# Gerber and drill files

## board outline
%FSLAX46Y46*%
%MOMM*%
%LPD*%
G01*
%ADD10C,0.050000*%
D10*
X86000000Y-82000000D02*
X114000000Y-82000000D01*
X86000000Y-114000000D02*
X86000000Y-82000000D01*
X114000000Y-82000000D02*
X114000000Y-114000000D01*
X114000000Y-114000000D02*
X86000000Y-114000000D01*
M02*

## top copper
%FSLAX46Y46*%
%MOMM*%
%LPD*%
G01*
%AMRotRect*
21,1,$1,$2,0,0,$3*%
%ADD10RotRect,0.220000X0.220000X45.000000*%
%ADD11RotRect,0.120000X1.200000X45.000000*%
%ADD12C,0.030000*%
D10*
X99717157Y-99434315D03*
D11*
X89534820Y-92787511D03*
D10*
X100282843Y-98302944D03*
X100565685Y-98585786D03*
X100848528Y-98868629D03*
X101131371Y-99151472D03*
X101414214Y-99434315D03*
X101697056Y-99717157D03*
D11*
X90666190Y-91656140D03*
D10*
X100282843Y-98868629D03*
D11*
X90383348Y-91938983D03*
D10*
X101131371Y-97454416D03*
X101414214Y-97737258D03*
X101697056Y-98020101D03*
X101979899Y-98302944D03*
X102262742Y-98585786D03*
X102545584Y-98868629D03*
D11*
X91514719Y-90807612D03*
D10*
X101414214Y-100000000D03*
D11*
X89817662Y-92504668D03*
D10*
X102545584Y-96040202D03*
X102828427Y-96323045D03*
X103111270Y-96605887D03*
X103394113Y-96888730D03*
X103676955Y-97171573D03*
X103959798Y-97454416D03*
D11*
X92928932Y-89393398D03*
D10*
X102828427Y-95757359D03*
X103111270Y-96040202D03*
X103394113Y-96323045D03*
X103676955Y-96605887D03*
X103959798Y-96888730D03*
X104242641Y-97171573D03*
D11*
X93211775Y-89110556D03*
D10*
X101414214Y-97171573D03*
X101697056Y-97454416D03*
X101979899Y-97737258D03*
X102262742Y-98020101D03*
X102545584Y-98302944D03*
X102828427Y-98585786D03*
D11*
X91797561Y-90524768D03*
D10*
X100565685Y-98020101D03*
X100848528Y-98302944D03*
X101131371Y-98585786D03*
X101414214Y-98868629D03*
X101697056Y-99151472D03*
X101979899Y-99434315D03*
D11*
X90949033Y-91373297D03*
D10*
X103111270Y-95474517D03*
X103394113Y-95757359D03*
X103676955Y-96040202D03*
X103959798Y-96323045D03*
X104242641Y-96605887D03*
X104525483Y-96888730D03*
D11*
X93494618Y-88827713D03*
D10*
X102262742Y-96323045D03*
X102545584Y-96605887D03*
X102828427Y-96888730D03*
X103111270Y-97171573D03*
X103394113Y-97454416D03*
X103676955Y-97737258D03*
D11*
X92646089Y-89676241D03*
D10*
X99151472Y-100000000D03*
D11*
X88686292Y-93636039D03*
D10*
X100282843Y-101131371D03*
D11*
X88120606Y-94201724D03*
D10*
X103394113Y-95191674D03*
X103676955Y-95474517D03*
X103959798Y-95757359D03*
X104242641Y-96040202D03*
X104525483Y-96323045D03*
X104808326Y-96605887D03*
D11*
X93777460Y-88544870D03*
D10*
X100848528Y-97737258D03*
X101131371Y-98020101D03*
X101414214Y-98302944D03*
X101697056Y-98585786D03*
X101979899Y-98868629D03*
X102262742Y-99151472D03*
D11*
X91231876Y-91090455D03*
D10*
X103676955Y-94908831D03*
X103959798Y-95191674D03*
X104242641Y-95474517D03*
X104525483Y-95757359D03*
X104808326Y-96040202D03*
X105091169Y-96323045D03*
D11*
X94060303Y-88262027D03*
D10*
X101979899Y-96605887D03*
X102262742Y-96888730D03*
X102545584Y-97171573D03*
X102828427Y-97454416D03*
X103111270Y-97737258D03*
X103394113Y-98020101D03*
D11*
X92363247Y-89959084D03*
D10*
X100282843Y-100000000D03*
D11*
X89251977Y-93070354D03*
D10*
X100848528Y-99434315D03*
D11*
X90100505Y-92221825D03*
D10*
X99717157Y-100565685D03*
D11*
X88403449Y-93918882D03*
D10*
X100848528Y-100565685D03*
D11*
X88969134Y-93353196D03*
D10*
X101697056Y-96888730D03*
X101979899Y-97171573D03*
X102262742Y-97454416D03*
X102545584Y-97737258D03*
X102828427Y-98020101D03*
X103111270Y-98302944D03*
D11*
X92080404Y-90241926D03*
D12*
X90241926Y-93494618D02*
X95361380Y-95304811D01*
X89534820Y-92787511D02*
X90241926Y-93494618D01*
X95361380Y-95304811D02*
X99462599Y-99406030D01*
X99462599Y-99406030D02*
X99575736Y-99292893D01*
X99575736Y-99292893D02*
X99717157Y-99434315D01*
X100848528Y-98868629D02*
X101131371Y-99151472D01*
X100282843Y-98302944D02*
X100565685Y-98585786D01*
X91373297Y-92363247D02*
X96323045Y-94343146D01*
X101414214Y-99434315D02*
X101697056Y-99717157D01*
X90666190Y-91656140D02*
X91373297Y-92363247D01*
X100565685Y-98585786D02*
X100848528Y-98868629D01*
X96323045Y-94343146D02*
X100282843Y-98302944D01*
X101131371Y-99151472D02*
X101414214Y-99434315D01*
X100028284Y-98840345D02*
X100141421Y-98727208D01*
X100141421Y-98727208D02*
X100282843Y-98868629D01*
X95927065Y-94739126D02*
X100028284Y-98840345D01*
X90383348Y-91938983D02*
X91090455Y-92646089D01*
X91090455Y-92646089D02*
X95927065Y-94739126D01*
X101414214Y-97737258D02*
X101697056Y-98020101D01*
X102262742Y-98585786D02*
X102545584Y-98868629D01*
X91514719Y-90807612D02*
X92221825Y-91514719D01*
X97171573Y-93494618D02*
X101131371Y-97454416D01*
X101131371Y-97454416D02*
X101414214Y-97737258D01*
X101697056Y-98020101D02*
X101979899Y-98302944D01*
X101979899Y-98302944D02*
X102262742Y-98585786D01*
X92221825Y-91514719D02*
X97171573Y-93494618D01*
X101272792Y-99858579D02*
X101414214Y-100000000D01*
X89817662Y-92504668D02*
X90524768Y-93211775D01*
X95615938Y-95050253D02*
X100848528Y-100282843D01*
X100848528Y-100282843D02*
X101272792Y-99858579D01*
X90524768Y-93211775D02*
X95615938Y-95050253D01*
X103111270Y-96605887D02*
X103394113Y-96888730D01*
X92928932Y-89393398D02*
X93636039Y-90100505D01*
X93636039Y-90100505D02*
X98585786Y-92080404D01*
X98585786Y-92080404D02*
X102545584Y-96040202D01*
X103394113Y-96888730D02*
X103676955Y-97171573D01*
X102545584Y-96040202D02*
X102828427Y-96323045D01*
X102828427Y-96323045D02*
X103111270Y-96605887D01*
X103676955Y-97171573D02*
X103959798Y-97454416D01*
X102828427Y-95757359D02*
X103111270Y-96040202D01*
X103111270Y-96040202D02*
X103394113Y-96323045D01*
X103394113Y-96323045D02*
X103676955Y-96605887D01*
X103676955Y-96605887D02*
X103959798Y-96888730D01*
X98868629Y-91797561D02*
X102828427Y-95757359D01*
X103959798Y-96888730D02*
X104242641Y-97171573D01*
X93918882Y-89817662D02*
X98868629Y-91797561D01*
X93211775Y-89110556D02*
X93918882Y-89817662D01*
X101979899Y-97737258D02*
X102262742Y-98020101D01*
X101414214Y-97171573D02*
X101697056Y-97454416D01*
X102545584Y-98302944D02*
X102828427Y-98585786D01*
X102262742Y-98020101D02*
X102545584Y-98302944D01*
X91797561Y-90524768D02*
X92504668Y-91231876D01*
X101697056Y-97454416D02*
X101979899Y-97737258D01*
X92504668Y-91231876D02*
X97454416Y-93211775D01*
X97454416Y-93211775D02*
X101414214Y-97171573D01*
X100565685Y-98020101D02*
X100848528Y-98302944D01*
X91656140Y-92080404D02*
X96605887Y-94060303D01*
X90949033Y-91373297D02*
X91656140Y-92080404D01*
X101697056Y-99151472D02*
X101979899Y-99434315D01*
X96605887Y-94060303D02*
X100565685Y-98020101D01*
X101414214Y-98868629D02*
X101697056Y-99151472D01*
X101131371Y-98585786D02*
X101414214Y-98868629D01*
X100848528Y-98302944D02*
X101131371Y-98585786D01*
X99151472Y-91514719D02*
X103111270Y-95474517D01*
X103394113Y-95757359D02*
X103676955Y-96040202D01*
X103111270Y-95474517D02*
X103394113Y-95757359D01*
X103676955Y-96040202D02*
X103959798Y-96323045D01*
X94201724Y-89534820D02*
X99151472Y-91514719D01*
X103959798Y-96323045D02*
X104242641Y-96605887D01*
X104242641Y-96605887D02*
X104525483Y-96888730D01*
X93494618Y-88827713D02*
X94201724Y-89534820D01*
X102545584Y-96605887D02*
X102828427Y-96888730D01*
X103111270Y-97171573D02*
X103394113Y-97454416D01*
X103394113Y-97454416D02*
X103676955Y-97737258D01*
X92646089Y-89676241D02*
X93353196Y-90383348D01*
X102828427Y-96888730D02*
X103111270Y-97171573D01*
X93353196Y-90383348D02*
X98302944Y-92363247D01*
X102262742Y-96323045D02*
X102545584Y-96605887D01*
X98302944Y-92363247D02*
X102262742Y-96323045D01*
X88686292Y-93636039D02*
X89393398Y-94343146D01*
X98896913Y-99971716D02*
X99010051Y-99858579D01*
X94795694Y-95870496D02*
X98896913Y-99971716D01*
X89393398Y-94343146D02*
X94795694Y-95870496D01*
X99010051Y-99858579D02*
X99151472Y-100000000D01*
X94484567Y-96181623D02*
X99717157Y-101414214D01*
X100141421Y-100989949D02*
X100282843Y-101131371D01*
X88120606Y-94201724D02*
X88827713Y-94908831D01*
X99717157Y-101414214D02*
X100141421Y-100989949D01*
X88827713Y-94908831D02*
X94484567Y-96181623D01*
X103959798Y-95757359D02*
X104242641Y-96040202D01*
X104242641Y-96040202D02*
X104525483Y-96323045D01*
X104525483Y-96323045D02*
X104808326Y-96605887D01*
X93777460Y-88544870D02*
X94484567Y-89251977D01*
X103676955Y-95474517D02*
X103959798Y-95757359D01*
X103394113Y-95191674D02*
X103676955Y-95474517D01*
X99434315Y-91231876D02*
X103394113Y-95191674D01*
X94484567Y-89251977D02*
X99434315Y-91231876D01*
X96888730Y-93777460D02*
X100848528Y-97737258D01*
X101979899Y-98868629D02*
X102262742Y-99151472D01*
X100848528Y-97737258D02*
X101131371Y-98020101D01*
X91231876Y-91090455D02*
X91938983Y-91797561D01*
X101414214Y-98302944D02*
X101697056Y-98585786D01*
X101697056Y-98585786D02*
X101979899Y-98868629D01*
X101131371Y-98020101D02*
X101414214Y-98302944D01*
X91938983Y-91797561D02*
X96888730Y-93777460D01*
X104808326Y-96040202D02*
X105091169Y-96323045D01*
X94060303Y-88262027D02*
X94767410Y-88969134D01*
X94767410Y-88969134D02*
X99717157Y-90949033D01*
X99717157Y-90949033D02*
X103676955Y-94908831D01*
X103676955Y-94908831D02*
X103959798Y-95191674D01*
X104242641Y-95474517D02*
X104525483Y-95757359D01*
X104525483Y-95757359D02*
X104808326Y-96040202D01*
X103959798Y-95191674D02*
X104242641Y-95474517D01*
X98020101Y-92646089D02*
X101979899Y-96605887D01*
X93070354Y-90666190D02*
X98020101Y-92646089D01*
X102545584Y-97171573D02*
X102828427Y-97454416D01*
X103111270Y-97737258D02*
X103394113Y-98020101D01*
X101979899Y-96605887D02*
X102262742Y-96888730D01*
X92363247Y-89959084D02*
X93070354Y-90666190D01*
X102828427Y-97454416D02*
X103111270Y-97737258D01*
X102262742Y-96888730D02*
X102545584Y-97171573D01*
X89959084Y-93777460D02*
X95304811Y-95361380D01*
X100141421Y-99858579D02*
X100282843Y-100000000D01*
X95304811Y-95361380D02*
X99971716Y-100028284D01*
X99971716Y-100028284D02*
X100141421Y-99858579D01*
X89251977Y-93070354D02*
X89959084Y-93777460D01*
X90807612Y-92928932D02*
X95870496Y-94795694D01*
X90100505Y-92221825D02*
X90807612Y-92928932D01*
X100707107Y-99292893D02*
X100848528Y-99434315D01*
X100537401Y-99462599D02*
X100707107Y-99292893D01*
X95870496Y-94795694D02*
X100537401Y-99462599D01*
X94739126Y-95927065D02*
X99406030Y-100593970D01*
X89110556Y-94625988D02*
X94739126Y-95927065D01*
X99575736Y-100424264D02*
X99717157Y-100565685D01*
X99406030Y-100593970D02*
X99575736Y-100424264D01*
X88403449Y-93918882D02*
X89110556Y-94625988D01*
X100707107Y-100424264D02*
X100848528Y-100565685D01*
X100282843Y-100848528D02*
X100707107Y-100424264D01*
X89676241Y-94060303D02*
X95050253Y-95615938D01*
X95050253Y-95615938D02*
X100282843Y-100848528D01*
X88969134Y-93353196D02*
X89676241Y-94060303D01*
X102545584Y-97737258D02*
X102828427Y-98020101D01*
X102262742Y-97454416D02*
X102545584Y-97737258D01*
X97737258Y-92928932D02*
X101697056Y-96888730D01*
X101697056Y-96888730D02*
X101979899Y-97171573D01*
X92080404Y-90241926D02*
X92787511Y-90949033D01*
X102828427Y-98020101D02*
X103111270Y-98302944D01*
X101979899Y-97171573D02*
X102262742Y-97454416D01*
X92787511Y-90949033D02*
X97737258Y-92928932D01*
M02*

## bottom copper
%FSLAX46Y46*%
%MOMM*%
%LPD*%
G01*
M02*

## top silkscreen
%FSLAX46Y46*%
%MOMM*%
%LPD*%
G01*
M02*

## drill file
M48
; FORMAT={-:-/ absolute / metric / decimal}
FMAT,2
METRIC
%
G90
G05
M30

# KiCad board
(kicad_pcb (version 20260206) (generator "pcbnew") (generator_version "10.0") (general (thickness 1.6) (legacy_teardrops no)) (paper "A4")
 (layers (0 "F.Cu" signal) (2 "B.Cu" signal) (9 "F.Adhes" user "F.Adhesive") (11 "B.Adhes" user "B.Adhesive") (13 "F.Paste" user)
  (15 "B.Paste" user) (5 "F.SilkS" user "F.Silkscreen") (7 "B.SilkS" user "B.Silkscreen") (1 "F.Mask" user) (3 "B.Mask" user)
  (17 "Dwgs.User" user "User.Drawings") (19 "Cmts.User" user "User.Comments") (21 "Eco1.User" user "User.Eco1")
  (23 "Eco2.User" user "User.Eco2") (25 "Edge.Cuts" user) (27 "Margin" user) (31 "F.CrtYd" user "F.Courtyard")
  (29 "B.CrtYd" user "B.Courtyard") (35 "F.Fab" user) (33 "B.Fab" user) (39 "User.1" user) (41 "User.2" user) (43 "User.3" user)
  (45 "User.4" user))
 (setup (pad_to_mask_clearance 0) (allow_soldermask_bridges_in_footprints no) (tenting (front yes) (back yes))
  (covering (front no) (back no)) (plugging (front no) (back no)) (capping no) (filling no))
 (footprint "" (layer "F.Cu") (at 0 0)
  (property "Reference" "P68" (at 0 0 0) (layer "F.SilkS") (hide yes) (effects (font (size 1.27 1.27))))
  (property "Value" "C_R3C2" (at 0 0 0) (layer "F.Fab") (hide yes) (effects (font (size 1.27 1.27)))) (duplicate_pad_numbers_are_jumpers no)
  (pad "1" connect rect (at 99.717157 99.434315 45) (size 0.22 0.22) (layers "F.Cu") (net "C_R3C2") (thermal_bridge_angle 45))
  (pad "2" connect rect (at 89.53482 92.787511 45) (size 0.12 1.2) (layers "F.Cu") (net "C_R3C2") (thermal_bridge_angle 45)))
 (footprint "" (layer "F.Cu") (at 0 0)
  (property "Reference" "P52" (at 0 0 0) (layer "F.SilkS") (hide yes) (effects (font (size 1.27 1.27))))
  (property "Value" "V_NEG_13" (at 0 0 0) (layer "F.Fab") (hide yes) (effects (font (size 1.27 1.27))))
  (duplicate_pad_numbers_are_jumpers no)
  (pad "1" connect rect (at 100.282843 98.302944 45) (size 0.22 0.22) (layers "F.Cu") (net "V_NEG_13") (thermal_bridge_angle 45))
  (pad "1" connect rect (at 100.565685 98.585786 45) (size 0.22 0.22) (layers "F.Cu") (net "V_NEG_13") (thermal_bridge_angle 45))
  (pad "1" connect rect (at 100.848528 98.868629 45) (size 0.22 0.22) (layers "F.Cu") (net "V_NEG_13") (thermal_bridge_angle 45))
  (pad "1" connect rect (at 101.131371 99.151472 45) (size 0.22 0.22) (layers "F.Cu") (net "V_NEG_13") (thermal_bridge_angle 45))
  (pad "1" connect rect (at 101.414214 99.434315 45) (size 0.22 0.22) (layers "F.Cu") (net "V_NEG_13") (thermal_bridge_angle 45))
  (pad "1" connect rect (at 101.697056 99.717157 45) (size 0.22 0.22) (layers "F.Cu") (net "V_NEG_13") (thermal_bridge_angle 45))
  (pad "2" connect rect (at 90.66619 91.65614 45) (size 0.12 1.2) (layers "F.Cu") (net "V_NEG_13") (thermal_bridge_angle 45)))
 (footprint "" (layer "F.Cu") (at 0 0)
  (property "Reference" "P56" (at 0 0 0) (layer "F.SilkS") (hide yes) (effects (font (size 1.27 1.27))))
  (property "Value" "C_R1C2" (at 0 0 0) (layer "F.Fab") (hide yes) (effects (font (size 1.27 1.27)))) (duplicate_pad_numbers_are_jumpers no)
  (pad "1" connect rect (at 100.282843 98.868629 45) (size 0.22 0.22) (layers "F.Cu") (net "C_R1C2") (thermal_bridge_angle 45))
  (pad "2" connect rect (at 90.383348 91.938983 45) (size 0.12 1.2) (layers "F.Cu") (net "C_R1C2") (thermal_bridge_angle 45)))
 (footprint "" (layer "F.Cu") (at 0 0)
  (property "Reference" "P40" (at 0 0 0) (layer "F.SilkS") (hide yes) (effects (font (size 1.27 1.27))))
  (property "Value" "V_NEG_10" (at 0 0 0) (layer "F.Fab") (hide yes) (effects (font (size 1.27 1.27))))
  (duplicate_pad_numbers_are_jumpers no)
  (pad "1" connect rect (at 101.131371 97.454416 45) (size 0.22 0.22) (layers "F.Cu") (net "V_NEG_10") (thermal_bridge_angle 45))
  (pad "1" connect rect (at 101.414214 97.737258 45) (size 0.22 0.22) (layers "F.Cu") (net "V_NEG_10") (thermal_bridge_angle 45))
  (pad "1" connect rect (at 101.697056 98.020101 45) (size 0.22 0.22) (layers "F.Cu") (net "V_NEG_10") (thermal_bridge_angle 45))
  (pad "1" connect rect (at 101.979899 98.302944 45) (size 0.22 0.22) (layers "F.Cu") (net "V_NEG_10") (thermal_bridge_angle 45))
  (pad "1" connect rect (at 102.262742 98.585786 45) (size 0.22 0.22) (layers "F.Cu") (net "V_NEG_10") (thermal_bridge_angle 45))
  (pad "1" connect rect (at 102.545584 98.868629 45) (size 0.22 0.22) (layers "F.Cu") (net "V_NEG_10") (thermal_bridge_angle 45))
  (pad "2" connect rect (at 91.514719 90.807612 45) (size 0.12 1.2) (layers "F.Cu") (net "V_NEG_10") (thermal_bridge_angle 45)))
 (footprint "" (layer "F.Cu") (at 0 0)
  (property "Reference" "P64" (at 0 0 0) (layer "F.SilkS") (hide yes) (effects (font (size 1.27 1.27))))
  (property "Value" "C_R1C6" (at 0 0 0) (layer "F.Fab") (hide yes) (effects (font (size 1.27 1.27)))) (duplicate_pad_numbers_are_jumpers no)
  (pad "1" connect rect (at 101.414214 100 45) (size 0.22 0.22) (layers "F.Cu") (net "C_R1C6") (thermal_bridge_angle 45))
  (pad "2" connect rect (at 89.817662 92.504668 45) (size 0.12 1.2) (layers "F.Cu") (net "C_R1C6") (thermal_bridge_angle 45)))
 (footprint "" (layer "F.Cu") (at 0 0)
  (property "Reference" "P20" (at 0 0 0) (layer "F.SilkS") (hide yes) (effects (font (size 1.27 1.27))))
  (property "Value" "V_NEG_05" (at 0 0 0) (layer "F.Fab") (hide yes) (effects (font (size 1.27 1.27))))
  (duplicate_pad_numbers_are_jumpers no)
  (pad "1" connect rect (at 102.545584 96.040202 45) (size 0.22 0.22) (layers "F.Cu") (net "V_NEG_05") (thermal_bridge_angle 45))
  (pad "1" connect rect (at 102.828427 96.323045 45) (size 0.22 0.22) (layers "F.Cu") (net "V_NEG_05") (thermal_bridge_angle 45))
  (pad "1" connect rect (at 103.11127 96.605887 45) (size 0.22 0.22) (layers "F.Cu") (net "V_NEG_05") (thermal_bridge_angle 45))
  (pad "1" connect rect (at 103.394113 96.88873 45) (size 0.22 0.22) (layers "F.Cu") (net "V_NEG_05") (thermal_bridge_angle 45))
  (pad "1" connect rect (at 103.676955 97.171573 45) (size 0.22 0.22) (layers "F.Cu") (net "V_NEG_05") (thermal_bridge_angle 45))
  (pad "1" connect rect (at 103.959798 97.454416 45) (size 0.22 0.22) (layers "F.Cu") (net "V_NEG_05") (thermal_bridge_angle 45))
  (pad "2" connect rect (at 92.928932 89.393398 45) (size 0.12 1.2) (layers "F.Cu") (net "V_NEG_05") (thermal_bridge_angle 45)))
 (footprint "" (layer "F.Cu") (at 0 0)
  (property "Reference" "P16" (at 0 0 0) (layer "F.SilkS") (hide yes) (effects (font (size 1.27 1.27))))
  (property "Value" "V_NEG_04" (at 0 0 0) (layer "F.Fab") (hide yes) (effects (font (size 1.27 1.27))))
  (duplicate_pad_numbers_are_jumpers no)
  (pad "1" connect rect (at 102.828427 95.757359 45) (size 0.22 0.22) (layers "F.Cu") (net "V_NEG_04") (thermal_bridge_angle 45))
  (pad "1" connect rect (at 103.11127 96.040202 45) (size 0.22 0.22) (layers "F.Cu") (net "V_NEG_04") (thermal_bridge_angle 45))
  (pad "1" connect rect (at 103.394113 96.323045 45) (size 0.22 0.22) (layers "F.Cu") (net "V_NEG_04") (thermal_bridge_angle 45))
  (pad "1" connect rect (at 103.676955 96.605887 45) (size 0.22 0.22) (layers "F.Cu") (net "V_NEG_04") (thermal_bridge_angle 45))
  (pad "1" connect rect (at 103.959798 96.88873 45) (size 0.22 0.22) (layers "F.Cu") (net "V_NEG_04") (thermal_bridge_angle 45))
  (pad "1" connect rect (at 104.242641 97.171573 45) (size 0.22 0.22) (layers "F.Cu") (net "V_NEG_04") (thermal_bridge_angle 45))
  (pad "2" connect rect (at 93.211775 89.110556 45) (size 0.12 1.2) (layers "F.Cu") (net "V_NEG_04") (thermal_bridge_angle 45)))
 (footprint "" (layer "F.Cu") (at 0 0)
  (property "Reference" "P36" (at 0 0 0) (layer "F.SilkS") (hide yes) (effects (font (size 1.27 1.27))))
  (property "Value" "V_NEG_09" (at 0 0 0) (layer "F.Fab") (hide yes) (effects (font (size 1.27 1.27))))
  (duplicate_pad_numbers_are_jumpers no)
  (pad "1" connect rect (at 101.414214 97.171573 45) (size 0.22 0.22) (layers "F.Cu") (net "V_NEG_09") (thermal_bridge_angle 45))
  (pad "1" connect rect (at 101.697056 97.454416 45) (size 0.22 0.22) (layers "F.Cu") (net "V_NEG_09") (thermal_bridge_angle 45))
  (pad "1" connect rect (at 101.979899 97.737258 45) (size 0.22 0.22) (layers "F.Cu") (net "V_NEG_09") (thermal_bridge_angle 45))
  (pad "1" connect rect (at 102.262742 98.020101 45) (size 0.22 0.22) (layers "F.Cu") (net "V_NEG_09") (thermal_bridge_angle 45))
  (pad "1" connect rect (at 102.545584 98.302944 45) (size 0.22 0.22) (layers "F.Cu") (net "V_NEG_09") (thermal_bridge_angle 45))
  (pad "1" connect rect (at 102.828427 98.585786 45) (size 0.22 0.22) (layers "F.Cu") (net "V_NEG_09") (thermal_bridge_angle 45))
  (pad "2" connect rect (at 91.797561 90.524768 45) (size 0.12 1.2) (layers "F.Cu") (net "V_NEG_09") (thermal_bridge_angle 45)))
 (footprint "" (layer "F.Cu") (at 0 0)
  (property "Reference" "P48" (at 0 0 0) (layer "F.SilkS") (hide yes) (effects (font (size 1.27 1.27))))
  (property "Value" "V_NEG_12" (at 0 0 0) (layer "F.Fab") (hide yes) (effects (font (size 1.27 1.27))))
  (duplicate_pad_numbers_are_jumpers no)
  (pad "1" connect rect (at 100.565685 98.020101 45) (size 0.22 0.22) (layers "F.Cu") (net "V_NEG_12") (thermal_bridge_angle 45))
  (pad "1" connect rect (at 100.848528 98.302944 45) (size 0.22 0.22) (layers "F.Cu") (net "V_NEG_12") (thermal_bridge_angle 45))
  (pad "1" connect rect (at 101.131371 98.585786 45) (size 0.22 0.22) (layers "F.Cu") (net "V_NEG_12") (thermal_bridge_angle 45))
  (pad "1" connect rect (at 101.414214 98.868629 45) (size 0.22 0.22) (layers "F.Cu") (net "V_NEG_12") (thermal_bridge_angle 45))
  (pad "1" connect rect (at 101.697056 99.151472 45) (size 0.22 0.22) (layers "F.Cu") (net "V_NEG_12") (thermal_bridge_angle 45))
  (pad "1" connect rect (at 101.979899 99.434315 45) (size 0.22 0.22) (layers "F.Cu") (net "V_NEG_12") (thermal_bridge_angle 45))
  (pad "2" connect rect (at 90.949033 91.373297 45) (size 0.12 1.2) (layers "F.Cu") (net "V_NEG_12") (thermal_bridge_angle 45)))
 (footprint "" (layer "F.Cu") (at 0 0)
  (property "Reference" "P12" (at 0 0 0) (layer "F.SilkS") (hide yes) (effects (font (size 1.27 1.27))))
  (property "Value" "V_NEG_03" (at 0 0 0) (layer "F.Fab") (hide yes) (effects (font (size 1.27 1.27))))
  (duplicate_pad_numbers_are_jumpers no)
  (pad "1" connect rect (at 103.11127 95.474517 45) (size 0.22 0.22) (layers "F.Cu") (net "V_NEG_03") (thermal_bridge_angle 45))
  (pad "1" connect rect (at 103.394113 95.757359 45) (size 0.22 0.22) (layers "F.Cu") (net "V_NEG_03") (thermal_bridge_angle 45))
  (pad "1" connect rect (at 103.676955 96.040202 45) (size 0.22 0.22) (layers "F.Cu") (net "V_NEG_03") (thermal_bridge_angle 45))
  (pad "1" connect rect (at 103.959798 96.323045 45) (size 0.22 0.22) (layers "F.Cu") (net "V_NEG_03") (thermal_bridge_angle 45))
  (pad "1" connect rect (at 104.242641 96.605887 45) (size 0.22 0.22) (layers "F.Cu") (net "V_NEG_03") (thermal_bridge_angle 45))
  (pad "1" connect rect (at 104.525483 96.88873 45) (size 0.22 0.22) (layers "F.Cu") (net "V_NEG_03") (thermal_bridge_angle 45))
  (pad "2" connect rect (at 93.494618 88.827713 45) (size 0.12 1.2) (layers "F.Cu") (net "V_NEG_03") (thermal_bridge_angle 45)))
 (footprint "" (layer "F.Cu") (at 0 0)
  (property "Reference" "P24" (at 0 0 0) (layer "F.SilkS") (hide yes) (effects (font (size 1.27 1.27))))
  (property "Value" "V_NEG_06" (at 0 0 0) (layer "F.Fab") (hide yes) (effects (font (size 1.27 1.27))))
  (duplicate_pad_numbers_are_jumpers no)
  (pad "1" connect rect (at 102.262742 96.323045 45) (size 0.22 0.22) (layers "F.Cu") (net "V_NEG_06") (thermal_bridge_angle 45))
  (pad "1" connect rect (at 102.545584 96.605887 45) (size 0.22 0.22) (layers "F.Cu") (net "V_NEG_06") (thermal_bridge_angle 45))
  (pad "1" connect rect (at 102.828427 96.88873 45) (size 0.22 0.22) (layers "F.Cu") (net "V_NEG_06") (thermal_bridge_angle 45))
  (pad "1" connect rect (at 103.11127 97.171573 45) (size 0.22 0.22) (layers "F.Cu") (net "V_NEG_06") (thermal_bridge_angle 45))
  (pad "1" connect rect (at 103.394113 97.454416 45) (size 0.22 0.22) (layers "F.Cu") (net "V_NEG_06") (thermal_bridge_angle 45))
  (pad "1" connect rect (at 103.676955 97.737258 45) (size 0.22 0.22) (layers "F.Cu") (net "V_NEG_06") (thermal_bridge_angle 45))
  (pad "2" connect rect (at 92.646089 89.676241 45) (size 0.12 1.2) (layers "F.Cu") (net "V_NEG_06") (thermal_bridge_angle 45)))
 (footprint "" (layer "F.Cu") (at 0 0)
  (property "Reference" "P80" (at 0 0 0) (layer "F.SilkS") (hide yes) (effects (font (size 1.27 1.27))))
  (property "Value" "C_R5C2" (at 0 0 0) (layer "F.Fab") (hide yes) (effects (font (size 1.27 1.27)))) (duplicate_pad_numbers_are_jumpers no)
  (pad "1" connect rect (at 99.151472 100 45) (size 0.22 0.22) (layers "F.Cu") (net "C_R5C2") (thermal_bridge_angle 45))
  (pad "2" connect rect (at 88.686292 93.636039 45) (size 0.12 1.2) (layers "F.Cu") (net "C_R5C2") (thermal_bridge_angle 45)))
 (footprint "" (layer "F.Cu") (at 0 0)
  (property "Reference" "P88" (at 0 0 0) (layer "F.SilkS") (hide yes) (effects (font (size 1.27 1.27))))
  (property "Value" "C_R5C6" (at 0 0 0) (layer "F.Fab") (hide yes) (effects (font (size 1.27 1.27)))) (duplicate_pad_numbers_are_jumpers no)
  (pad "1" connect rect (at 100.282843 101.131371 45) (size 0.22 0.22) (layers "F.Cu") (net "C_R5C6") (thermal_bridge_angle 45))
  (pad "2" connect rect (at 88.120606 94.201724 45) (size 0.12 1.2) (layers "F.Cu") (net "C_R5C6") (thermal_bridge_angle 45)))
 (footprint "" (layer "F.Cu") (at 0 0)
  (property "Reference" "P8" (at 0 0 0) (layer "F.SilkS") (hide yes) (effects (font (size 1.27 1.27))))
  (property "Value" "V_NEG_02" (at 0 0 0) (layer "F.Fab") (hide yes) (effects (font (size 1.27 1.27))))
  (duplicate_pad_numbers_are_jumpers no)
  (pad "1" connect rect (at 103.394113 95.191674 45) (size 0.22 0.22) (layers "F.Cu") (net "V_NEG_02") (thermal_bridge_angle 45))
  (pad "1" connect rect (at 103.676955 95.474517 45) (size 0.22 0.22) (layers "F.Cu") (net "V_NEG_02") (thermal_bridge_angle 45))
  (pad "1" connect rect (at 103.959798 95.757359 45) (size 0.22 0.22) (layers "F.Cu") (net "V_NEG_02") (thermal_bridge_angle 45))
  (pad "1" connect rect (at 104.242641 96.040202 45) (size 0.22 0.22) (layers "F.Cu") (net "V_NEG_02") (thermal_bridge_angle 45))
  (pad "1" connect rect (at 104.525483 96.323045 45) (size 0.22 0.22) (layers "F.Cu") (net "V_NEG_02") (thermal_bridge_angle 45))
  (pad "1" connect rect (at 104.808326 96.605887 45) (size 0.22 0.22) (layers "F.Cu") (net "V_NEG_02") (thermal_bridge_angle 45))
  (pad "2" connect rect (at 93.77746 88.54487 45) (size 0.12 1.2) (layers "F.Cu") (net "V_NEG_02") (thermal_bridge_angle 45)))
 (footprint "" (layer "F.Cu") (at 0 0)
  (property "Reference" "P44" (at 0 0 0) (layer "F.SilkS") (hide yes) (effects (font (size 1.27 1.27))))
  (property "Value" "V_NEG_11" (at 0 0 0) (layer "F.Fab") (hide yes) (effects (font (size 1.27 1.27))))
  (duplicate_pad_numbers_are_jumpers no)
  (pad "1" connect rect (at 100.848528 97.737258 45) (size 0.22 0.22) (layers "F.Cu") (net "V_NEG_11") (thermal_bridge_angle 45))
  (pad "1" connect rect (at 101.131371 98.020101 45) (size 0.22 0.22) (layers "F.Cu") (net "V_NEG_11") (thermal_bridge_angle 45))
  (pad "1" connect rect (at 101.414214 98.302944 45) (size 0.22 0.22) (layers "F.Cu") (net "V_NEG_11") (thermal_bridge_angle 45))
  (pad "1" connect rect (at 101.697056 98.585786 45) (size 0.22 0.22) (layers "F.Cu") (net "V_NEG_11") (thermal_bridge_angle 45))
  (pad "1" connect rect (at 101.979899 98.868629 45) (size 0.22 0.22) (layers "F.Cu") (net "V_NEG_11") (thermal_bridge_angle 45))
  (pad "1" connect rect (at 102.262742 99.151472 45) (size 0.22 0.22) (layers "F.Cu") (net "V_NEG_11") (thermal_bridge_angle 45))
  (pad "2" connect rect (at 91.231876 91.090455 45) (size 0.12 1.2) (layers "F.Cu") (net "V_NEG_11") (thermal_bridge_angle 45)))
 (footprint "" (layer "F.Cu") (at 0 0)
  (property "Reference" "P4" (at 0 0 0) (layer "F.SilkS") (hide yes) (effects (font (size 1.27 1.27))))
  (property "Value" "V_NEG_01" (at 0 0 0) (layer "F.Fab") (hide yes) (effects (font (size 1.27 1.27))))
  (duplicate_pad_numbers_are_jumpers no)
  (pad "1" connect rect (at 103.676955 94.908831 45) (size 0.22 0.22) (layers "F.Cu") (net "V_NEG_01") (thermal_bridge_angle 45))
  (pad "1" connect rect (at 103.959798 95.191674 45) (size 0.22 0.22) (layers "F.Cu") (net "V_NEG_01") (thermal_bridge_angle 45))
  (pad "1" connect rect (at 104.242641 95.474517 45) (size 0.22 0.22) (layers "F.Cu") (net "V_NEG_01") (thermal_bridge_angle 45))
  (pad "1" connect rect (at 104.525483 95.757359 45) (size 0.22 0.22) (layers "F.Cu") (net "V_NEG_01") (thermal_bridge_angle 45))
  (pad "1" connect rect (at 104.808326 96.040202 45) (size 0.22 0.22) (layers "F.Cu") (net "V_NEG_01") (thermal_bridge_angle 45))
  (pad "1" connect rect (at 105.091169 96.323045 45) (size 0.22 0.22) (layers "F.Cu") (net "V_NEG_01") (thermal_bridge_angle 45))
  (pad "2" connect rect (at 94.060303 88.262027 45) (size 0.12 1.2) (layers "F.Cu") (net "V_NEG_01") (thermal_bridge_angle 45)))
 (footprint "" (layer "F.Cu") (at 0 0)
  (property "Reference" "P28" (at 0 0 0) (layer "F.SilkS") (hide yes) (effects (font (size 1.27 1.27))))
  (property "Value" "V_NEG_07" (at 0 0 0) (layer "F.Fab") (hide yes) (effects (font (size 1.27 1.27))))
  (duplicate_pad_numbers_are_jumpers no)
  (pad "1" connect rect (at 101.979899 96.605887 45) (size 0.22 0.22) (layers "F.Cu") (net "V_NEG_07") (thermal_bridge_angle 45))
  (pad "1" connect rect (at 102.262742 96.88873 45) (size 0.22 0.22) (layers "F.Cu") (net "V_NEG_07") (thermal_bridge_angle 45))
  (pad "1" connect rect (at 102.545584 97.171573 45) (size 0.22 0.22) (layers "F.Cu") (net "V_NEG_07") (thermal_bridge_angle 45))
  (pad "1" connect rect (at 102.828427 97.454416 45) (size 0.22 0.22) (layers "F.Cu") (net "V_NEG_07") (thermal_bridge_angle 45))
  (pad "1" connect rect (at 103.11127 97.737258 45) (size 0.22 0.22) (layers "F.Cu") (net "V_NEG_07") (thermal_bridge_angle 45))
  (pad "1" connect rect (at 103.394113 98.020101 45) (size 0.22 0.22) (layers "F.Cu") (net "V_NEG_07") (thermal_bridge_angle 45))
  (pad "2" connect rect (at 92.363247 89.959084 45) (size 0.12 1.2) (layers "F.Cu") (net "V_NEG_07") (thermal_bridge_angle 45)))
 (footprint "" (layer "F.Cu") (at 0 0)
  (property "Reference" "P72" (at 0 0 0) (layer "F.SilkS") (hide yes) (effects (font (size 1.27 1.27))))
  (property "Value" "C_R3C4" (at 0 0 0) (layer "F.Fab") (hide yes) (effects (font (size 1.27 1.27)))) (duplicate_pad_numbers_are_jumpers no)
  (pad "1" connect rect (at 100.282843 100 45) (size 0.22 0.22) (layers "F.Cu") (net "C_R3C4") (thermal_bridge_angle 45))
  (pad "2" connect rect (at 89.251977 93.070354 45) (size 0.12 1.2) (layers "F.Cu") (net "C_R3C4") (thermal_bridge_angle 45)))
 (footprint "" (layer "F.Cu") (at 0 0)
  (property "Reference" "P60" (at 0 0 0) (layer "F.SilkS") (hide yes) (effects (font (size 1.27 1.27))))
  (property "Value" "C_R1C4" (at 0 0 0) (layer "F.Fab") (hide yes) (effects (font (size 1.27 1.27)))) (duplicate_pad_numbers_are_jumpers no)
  (pad "1" connect rect (at 100.848528 99.434315 45) (size 0.22 0.22) (layers "F.Cu") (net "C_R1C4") (thermal_bridge_angle 45))
  (pad "2" connect rect (at 90.100505 92.221825 45) (size 0.12 1.2) (layers "F.Cu") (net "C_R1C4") (thermal_bridge_angle 45)))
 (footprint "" (layer "F.Cu") (at 0 0)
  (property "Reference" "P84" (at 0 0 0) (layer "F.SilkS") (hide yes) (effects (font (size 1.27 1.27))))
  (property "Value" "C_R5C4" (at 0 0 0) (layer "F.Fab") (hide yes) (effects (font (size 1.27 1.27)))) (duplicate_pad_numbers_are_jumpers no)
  (pad "1" connect rect (at 99.717157 100.565685 45) (size 0.22 0.22) (layers "F.Cu") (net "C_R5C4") (thermal_bridge_angle 45))
  (pad "2" connect rect (at 88.403449 93.918882 45) (size 0.12 1.2) (layers "F.Cu") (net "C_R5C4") (thermal_bridge_angle 45)))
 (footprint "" (layer "F.Cu") (at 0 0)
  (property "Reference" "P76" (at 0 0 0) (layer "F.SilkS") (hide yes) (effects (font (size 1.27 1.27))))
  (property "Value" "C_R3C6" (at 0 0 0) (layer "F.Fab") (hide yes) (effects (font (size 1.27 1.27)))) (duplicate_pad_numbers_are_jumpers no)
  (pad "1" connect rect (at 100.848528 100.565685 45) (size 0.22 0.22) (layers "F.Cu") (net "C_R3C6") (thermal_bridge_angle 45))
  (pad "2" connect rect (at 88.969134 93.353196 45) (size 0.12 1.2) (layers "F.Cu") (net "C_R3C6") (thermal_bridge_angle 45)))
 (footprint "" (layer "F.Cu") (at 0 0)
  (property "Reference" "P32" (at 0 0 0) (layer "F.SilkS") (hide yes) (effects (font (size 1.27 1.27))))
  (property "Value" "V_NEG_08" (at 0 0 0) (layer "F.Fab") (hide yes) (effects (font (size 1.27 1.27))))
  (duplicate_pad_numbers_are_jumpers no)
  (pad "1" connect rect (at 101.697056 96.88873 45) (size 0.22 0.22) (layers "F.Cu") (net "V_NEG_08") (thermal_bridge_angle 45))
  (pad "1" connect rect (at 101.979899 97.171573 45) (size 0.22 0.22) (layers "F.Cu") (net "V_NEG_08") (thermal_bridge_angle 45))
  (pad "1" connect rect (at 102.262742 97.454416 45) (size 0.22 0.22) (layers "F.Cu") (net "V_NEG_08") (thermal_bridge_angle 45))
  (pad "1" connect rect (at 102.545584 97.737258 45) (size 0.22 0.22) (layers "F.Cu") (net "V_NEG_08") (thermal_bridge_angle 45))
  (pad "1" connect rect (at 102.828427 98.020101 45) (size 0.22 0.22) (layers "F.Cu") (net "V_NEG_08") (thermal_bridge_angle 45))
  (pad "1" connect rect (at 103.11127 98.302944 45) (size 0.22 0.22) (layers "F.Cu") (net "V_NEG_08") (thermal_bridge_angle 45))
  (pad "2" connect rect (at 92.080404 90.241926 45) (size 0.12 1.2) (layers "F.Cu") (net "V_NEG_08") (thermal_bridge_angle 45)))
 (gr_line (start 86 82) (end 114 82) (stroke (width 0.05) (type default)) (layer "Edge.Cuts"))
 (gr_line (start 86 114) (end 86 82) (stroke (width 0.05) (type default)) (layer "Edge.Cuts"))
 (gr_line (start 114 82) (end 114 114) (stroke (width 0.05) (type default)) (layer "Edge.Cuts"))
 (gr_line (start 114 114) (end 86 114) (stroke (width 0.05) (type default)) (layer "Edge.Cuts"))
 (segment (start 90.241926 93.494618) (end 95.36138 95.304811) (width 0.03) (layer "F.Cu") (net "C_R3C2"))
 (segment (start 89.53482 92.787511) (end 90.241926 93.494618) (width 0.03) (layer "F.Cu") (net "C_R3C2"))
 (segment (start 95.36138 95.304811) (end 99.462599 99.40603) (width 0.03) (layer "F.Cu") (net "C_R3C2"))
 (segment (start 99.462599 99.40603) (end 99.575736 99.292893) (width 0.03) (layer "F.Cu") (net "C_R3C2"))
 (segment (start 99.575736 99.292893) (end 99.717157 99.434315) (width 0.03) (layer "F.Cu") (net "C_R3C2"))
 (segment (start 100.848528 98.868629) (end 101.131371 99.151472) (width 0.03) (layer "F.Cu") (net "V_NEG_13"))
 (segment (start 100.282843 98.302944) (end 100.565685 98.585786) (width 0.03) (layer "F.Cu") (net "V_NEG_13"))
 (segment (start 91.373297 92.363247) (end 96.323045 94.343146) (width 0.03) (layer "F.Cu") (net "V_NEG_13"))
 (segment (start 101.414214 99.434315) (end 101.697056 99.717157) (width 0.03) (layer "F.Cu") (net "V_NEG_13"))
 (segment (start 90.66619 91.65614) (end 91.373297 92.363247) (width 0.03) (layer "F.Cu") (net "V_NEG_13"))
 (segment (start 100.565685 98.585786) (end 100.848528 98.868629) (width 0.03) (layer "F.Cu") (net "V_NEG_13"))
 (segment (start 96.323045 94.343146) (end 100.282843 98.302944) (width 0.03) (layer "F.Cu") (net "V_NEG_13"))
 (segment (start 101.131371 99.151472) (end 101.414214 99.434315) (width 0.03) (layer "F.Cu") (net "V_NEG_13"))
 (segment (start 100.028284 98.840345) (end 100.141421 98.727208) (width 0.03) (layer "F.Cu") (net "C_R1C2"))
 (segment (start 100.141421 98.727208) (end 100.282843 98.868629) (width 0.03) (layer "F.Cu") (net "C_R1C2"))
 (segment (start 95.927065 94.739126) (end 100.028284 98.840345) (width 0.03) (layer "F.Cu") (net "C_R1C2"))
 (segment (start 90.383348 91.938983) (end 91.090455 92.646089) (width 0.03) (layer "F.Cu") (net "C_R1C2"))
 (segment (start 91.090455 92.646089) (end 95.927065 94.739126) (width 0.03) (layer "F.Cu") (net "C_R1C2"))
 (segment (start 101.414214 97.737258) (end 101.697056 98.020101) (width 0.03) (layer "F.Cu") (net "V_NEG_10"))
 (segment (start 102.262742 98.585786) (end 102.545584 98.868629) (width 0.03) (layer "F.Cu") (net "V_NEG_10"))
 (segment (start 91.514719 90.807612) (end 92.221825 91.514719) (width 0.03) (layer "F.Cu") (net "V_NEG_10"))
 (segment (start 97.171573 93.494618) (end 101.131371 97.454416) (width 0.03) (layer "F.Cu") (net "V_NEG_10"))
 (segment (start 101.131371 97.454416) (end 101.414214 97.737258) (width 0.03) (layer "F.Cu") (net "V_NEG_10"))
 (segment (start 101.697056 98.020101) (end 101.979899 98.302944) (width 0.03) (layer "F.Cu") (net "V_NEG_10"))
 (segment (start 101.979899 98.302944) (end 102.262742 98.585786) (width 0.03) (layer "F.Cu") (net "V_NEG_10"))
 (segment (start 92.221825 91.514719) (end 97.171573 93.494618) (width 0.03) (layer "F.Cu") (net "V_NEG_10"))
 (segment (start 101.272792 99.858579) (end 101.414214 100) (width 0.03) (layer "F.Cu") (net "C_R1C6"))
 (segment (start 89.817662 92.504668) (end 90.524768 93.211775) (width 0.03) (layer "F.Cu") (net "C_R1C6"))
 (segment (start 95.615938 95.050253) (end 100.848528 100.282843) (width 0.03) (layer "F.Cu") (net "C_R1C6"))
 (segment (start 100.848528 100.282843) (end 101.272792 99.858579) (width 0.03) (layer "F.Cu") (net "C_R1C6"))
 (segment (start 90.524768 93.211775) (end 95.615938 95.050253) (width 0.03) (layer "F.Cu") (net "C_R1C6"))
 (segment (start 103.11127 96.605887) (end 103.394113 96.88873) (width 0.03) (layer "F.Cu") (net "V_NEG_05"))
 (segment (start 92.928932 89.393398) (end 93.636039 90.100505) (width 0.03) (layer "F.Cu") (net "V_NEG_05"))
 (segment (start 93.636039 90.100505) (end 98.585786 92.080404) (width 0.03) (layer "F.Cu") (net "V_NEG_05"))
 (segment (start 98.585786 92.080404) (end 102.545584 96.040202) (width 0.03) (layer "F.Cu") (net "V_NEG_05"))
 (segment (start 103.394113 96.88873) (end 103.676955 97.171573) (width 0.03) (layer "F.Cu") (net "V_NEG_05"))
 (segment (start 102.545584 96.040202) (end 102.828427 96.323045) (width 0.03) (layer "F.Cu") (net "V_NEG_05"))
 (segment (start 102.828427 96.323045) (end 103.11127 96.605887) (width 0.03) (layer "F.Cu") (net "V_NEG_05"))
 (segment (start 103.676955 97.171573) (end 103.959798 97.454416) (width 0.03) (layer "F.Cu") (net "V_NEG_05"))
 (segment (start 102.828427 95.757359) (end 103.11127 96.040202) (width 0.03) (layer "F.Cu") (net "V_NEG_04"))
 (segment (start 103.11127 96.040202) (end 103.394113 96.323045) (width 0.03) (layer "F.Cu") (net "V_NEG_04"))
 (segment (start 103.394113 96.323045) (end 103.676955 96.605887) (width 0.03) (layer "F.Cu") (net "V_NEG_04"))
 (segment (start 103.676955 96.605887) (end 103.959798 96.88873) (width 0.03) (layer "F.Cu") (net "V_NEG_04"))
 (segment (start 98.868629 91.797561) (end 102.828427 95.757359) (width 0.03) (layer "F.Cu") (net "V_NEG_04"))
 (segment (start 103.959798 96.88873) (end 104.242641 97.171573) (width 0.03) (layer "F.Cu") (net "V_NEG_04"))
 (segment (start 93.918882 89.817662) (end 98.868629 91.797561) (width 0.03) (layer "F.Cu") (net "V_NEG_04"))
 (segment (start 93.211775 89.110556) (end 93.918882 89.817662) (width 0.03) (layer "F.Cu") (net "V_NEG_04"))
 (segment (start 101.979899 97.737258) (end 102.262742 98.020101) (width 0.03) (layer "F.Cu") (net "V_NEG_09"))
 (segment (start 101.414214 97.171573) (end 101.697056 97.454416) (width 0.03) (layer "F.Cu") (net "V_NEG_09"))
 (segment (start 102.545584 98.302944) (end 102.828427 98.585786) (width 0.03) (layer "F.Cu") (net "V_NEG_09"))
 (segment (start 102.262742 98.020101) (end 102.545584 98.302944) (width 0.03) (layer "F.Cu") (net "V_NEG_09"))
 (segment (start 91.797561 90.524768) (end 92.504668 91.231876) (width 0.03) (layer "F.Cu") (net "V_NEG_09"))
 (segment (start 101.697056 97.454416) (end 101.979899 97.737258) (width 0.03) (layer "F.Cu") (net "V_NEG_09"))
 (segment (start 92.504668 91.231876) (end 97.454416 93.211775) (width 0.03) (layer "F.Cu") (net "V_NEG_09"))
 (segment (start 97.454416 93.211775) (end 101.414214 97.171573) (width 0.03) (layer "F.Cu") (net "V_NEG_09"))
 (segment (start 100.565685 98.020101) (end 100.848528 98.302944) (width 0.03) (layer "F.Cu") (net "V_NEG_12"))
 (segment (start 91.65614 92.080404) (end 96.605887 94.060303) (width 0.03) (layer "F.Cu") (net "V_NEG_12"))
 (segment (start 90.949033 91.373297) (end 91.65614 92.080404) (width 0.03) (layer "F.Cu") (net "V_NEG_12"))
 (segment (start 101.697056 99.151472) (end 101.979899 99.434315) (width 0.03) (layer "F.Cu") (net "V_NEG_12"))
 (segment (start 96.605887 94.060303) (end 100.565685 98.020101) (width 0.03) (layer "F.Cu") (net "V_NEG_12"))
 (segment (start 101.414214 98.868629) (end 101.697056 99.151472) (width 0.03) (layer "F.Cu") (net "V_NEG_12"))
 (segment (start 101.131371 98.585786) (end 101.414214 98.868629) (width 0.03) (layer "F.Cu") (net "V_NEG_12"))
 (segment (start 100.848528 98.302944) (end 101.131371 98.585786) (width 0.03) (layer "F.Cu") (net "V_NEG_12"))
 (segment (start 99.151472 91.514719) (end 103.11127 95.474517) (width 0.03) (layer "F.Cu") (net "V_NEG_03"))
 (segment (start 103.394113 95.757359) (end 103.676955 96.040202) (width 0.03) (layer "F.Cu") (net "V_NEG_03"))
 (segment (start 103.11127 95.474517) (end 103.394113 95.757359) (width 0.03) (layer "F.Cu") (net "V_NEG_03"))
 (segment (start 103.676955 96.040202) (end 103.959798 96.323045) (width 0.03) (layer "F.Cu") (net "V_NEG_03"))
 (segment (start 94.201724 89.53482) (end 99.151472 91.514719) (width 0.03) (layer "F.Cu") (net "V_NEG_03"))
 (segment (start 103.959798 96.323045) (end 104.242641 96.605887) (width 0.03) (layer "F.Cu") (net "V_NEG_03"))
 (segment (start 104.242641 96.605887) (end 104.525483 96.88873) (width 0.03) (layer "F.Cu") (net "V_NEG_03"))
 (segment (start 93.494618 88.827713) (end 94.201724 89.53482) (width 0.03) (layer "F.Cu") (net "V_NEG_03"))
 (segment (start 102.545584 96.605887) (end 102.828427 96.88873) (width 0.03) (layer "F.Cu") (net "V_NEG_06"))
 (segment (start 103.11127 97.171573) (end 103.394113 97.454416) (width 0.03) (layer "F.Cu") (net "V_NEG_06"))
 (segment (start 103.394113 97.454416) (end 103.676955 97.737258) (width 0.03) (layer "F.Cu") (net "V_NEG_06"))
 (segment (start 92.646089 89.676241) (end 93.353196 90.383348) (width 0.03) (layer "F.Cu") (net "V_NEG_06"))
 (segment (start 102.828427 96.88873) (end 103.11127 97.171573) (width 0.03) (layer "F.Cu") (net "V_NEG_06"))
 (segment (start 93.353196 90.383348) (end 98.302944 92.363247) (width 0.03) (layer "F.Cu") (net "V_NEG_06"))
 (segment (start 102.262742 96.323045) (end 102.545584 96.605887) (width 0.03) (layer "F.Cu") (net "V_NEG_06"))
 (segment (start 98.302944 92.363247) (end 102.262742 96.323045) (width 0.03) (layer "F.Cu") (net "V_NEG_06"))
 (segment (start 88.686292 93.636039) (end 89.393398 94.343146) (width 0.03) (layer "F.Cu") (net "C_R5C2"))
 (segment (start 98.896913 99.971716) (end 99.010051 99.858579) (width 0.03) (layer "F.Cu") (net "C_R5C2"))
 (segment (start 94.795694 95.870496) (end 98.896913 99.971716) (width 0.03) (layer "F.Cu") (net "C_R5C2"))
 (segment (start 89.393398 94.343146) (end 94.795694 95.870496) (width 0.03) (layer "F.Cu") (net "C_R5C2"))
 (segment (start 99.010051 99.858579) (end 99.151472 100) (width 0.03) (layer "F.Cu") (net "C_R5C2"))
 (segment (start 94.484567 96.181623) (end 99.717157 101.414214) (width 0.03) (layer "F.Cu") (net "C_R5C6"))
 (segment (start 100.141421 100.989949) (end 100.282843 101.131371) (width 0.03) (layer "F.Cu") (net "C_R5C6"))
 (segment (start 88.120606 94.201724) (end 88.827713 94.908831) (width 0.03) (layer "F.Cu") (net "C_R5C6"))
 (segment (start 99.717157 101.414214) (end 100.141421 100.989949) (width 0.03) (layer "F.Cu") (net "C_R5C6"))
 (segment (start 88.827713 94.908831) (end 94.484567 96.181623) (width 0.03) (layer "F.Cu") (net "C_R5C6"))
 (segment (start 103.959798 95.757359) (end 104.242641 96.040202) (width 0.03) (layer "F.Cu") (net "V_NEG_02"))
 (segment (start 104.242641 96.040202) (end 104.525483 96.323045) (width 0.03) (layer "F.Cu") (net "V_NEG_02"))
 (segment (start 104.525483 96.323045) (end 104.808326 96.605887) (width 0.03) (layer "F.Cu") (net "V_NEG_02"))
 (segment (start 93.77746 88.54487) (end 94.484567 89.251977) (width 0.03) (layer "F.Cu") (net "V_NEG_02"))
 (segment (start 103.676955 95.474517) (end 103.959798 95.757359) (width 0.03) (layer "F.Cu") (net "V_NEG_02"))
 (segment (start 103.394113 95.191674) (end 103.676955 95.474517) (width 0.03) (layer "F.Cu") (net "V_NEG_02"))
 (segment (start 99.434315 91.231876) (end 103.394113 95.191674) (width 0.03) (layer "F.Cu") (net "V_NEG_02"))
 (segment (start 94.484567 89.251977) (end 99.434315 91.231876) (width 0.03) (layer "F.Cu") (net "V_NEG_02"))
 (segment (start 96.88873 93.77746) (end 100.848528 97.737258) (width 0.03) (layer "F.Cu") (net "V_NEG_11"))
 (segment (start 101.979899 98.868629) (end 102.262742 99.151472) (width 0.03) (layer "F.Cu") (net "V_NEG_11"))
 (segment (start 100.848528 97.737258) (end 101.131371 98.020101) (width 0.03) (layer "F.Cu") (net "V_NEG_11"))
 (segment (start 91.231876 91.090455) (end 91.938983 91.797561) (width 0.03) (layer "F.Cu") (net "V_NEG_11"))
 (segment (start 101.414214 98.302944) (end 101.697056 98.585786) (width 0.03) (layer "F.Cu") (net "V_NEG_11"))
 (segment (start 101.697056 98.585786) (end 101.979899 98.868629) (width 0.03) (layer "F.Cu") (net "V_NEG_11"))
 (segment (start 101.131371 98.020101) (end 101.414214 98.302944) (width 0.03) (layer "F.Cu") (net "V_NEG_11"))
 (segment (start 91.938983 91.797561) (end 96.88873 93.77746) (width 0.03) (layer "F.Cu") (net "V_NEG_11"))
 (segment (start 104.808326 96.040202) (end 105.091169 96.323045) (width 0.03) (layer "F.Cu") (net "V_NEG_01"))
 (segment (start 94.060303 88.262027) (end 94.76741 88.969134) (width 0.03) (layer "F.Cu") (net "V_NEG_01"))
 (segment (start 94.76741 88.969134) (end 99.717157 90.949033) (width 0.03) (layer "F.Cu") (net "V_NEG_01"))
 (segment (start 99.717157 90.949033) (end 103.676955 94.908831) (width 0.03) (layer "F.Cu") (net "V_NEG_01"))
 (segment (start 103.676955 94.908831) (end 103.959798 95.191674) (width 0.03) (layer "F.Cu") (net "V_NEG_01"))
 (segment (start 104.242641 95.474517) (end 104.525483 95.757359) (width 0.03) (layer "F.Cu") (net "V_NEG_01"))
 (segment (start 104.525483 95.757359) (end 104.808326 96.040202) (width 0.03) (layer "F.Cu") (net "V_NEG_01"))
 (segment (start 103.959798 95.191674) (end 104.242641 95.474517) (width 0.03) (layer "F.Cu") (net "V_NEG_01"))
 (segment (start 98.020101 92.646089) (end 101.979899 96.605887) (width 0.03) (layer "F.Cu") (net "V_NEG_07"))
 (segment (start 93.070354 90.66619) (end 98.020101 92.646089) (width 0.03) (layer "F.Cu") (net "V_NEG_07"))
 (segment (start 102.545584 97.171573) (end 102.828427 97.454416) (width 0.03) (layer "F.Cu") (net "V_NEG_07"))
 (segment (start 103.11127 97.737258) (end 103.394113 98.020101) (width 0.03) (layer "F.Cu") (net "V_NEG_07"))
 (segment (start 101.979899 96.605887) (end 102.262742 96.88873) (width 0.03) (layer "F.Cu") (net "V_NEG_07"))
 (segment (start 92.363247 89.959084) (end 93.070354 90.66619) (width 0.03) (layer "F.Cu") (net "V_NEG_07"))
 (segment (start 102.828427 97.454416) (end 103.11127 97.737258) (width 0.03) (layer "F.Cu") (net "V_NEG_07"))
 (segment (start 102.262742 96.88873) (end 102.545584 97.171573) (width 0.03) (layer "F.Cu") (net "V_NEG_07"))
 (segment (start 89.959084 93.77746) (end 95.304811 95.36138) (width 0.03) (layer "F.Cu") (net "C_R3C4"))
 (segment (start 100.141421 99.858579) (end 100.282843 100) (width 0.03) (layer "F.Cu") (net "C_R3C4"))
 (segment (start 95.304811 95.36138) (end 99.971716 100.028284) (width 0.03) (layer "F.Cu") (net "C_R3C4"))
 (segment (start 99.971716 100.028284) (end 100.141421 99.858579) (width 0.03) (layer "F.Cu") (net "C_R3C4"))
 (segment (start 89.251977 93.070354) (end 89.959084 93.77746) (width 0.03) (layer "F.Cu") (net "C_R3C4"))
 (segment (start 90.807612 92.928932) (end 95.870496 94.795694) (width 0.03) (layer "F.Cu") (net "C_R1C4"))
 (segment (start 90.100505 92.221825) (end 90.807612 92.928932) (width 0.03) (layer "F.Cu") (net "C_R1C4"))
 (segment (start 100.707107 99.292893) (end 100.848528 99.434315) (width 0.03) (layer "F.Cu") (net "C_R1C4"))
 (segment (start 100.537401 99.462599) (end 100.707107 99.292893) (width 0.03) (layer "F.Cu") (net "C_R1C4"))
 (segment (start 95.870496 94.795694) (end 100.537401 99.462599) (width 0.03) (layer "F.Cu") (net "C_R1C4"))
 (segment (start 94.739126 95.927065) (end 99.40603 100.59397) (width 0.03) (layer "F.Cu") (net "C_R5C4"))
 (segment (start 89.110556 94.625988) (end 94.739126 95.927065) (width 0.03) (layer "F.Cu") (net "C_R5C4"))
 (segment (start 99.575736 100.424264) (end 99.717157 100.565685) (width 0.03) (layer "F.Cu") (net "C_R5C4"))
 (segment (start 99.40603 100.59397) (end 99.575736 100.424264) (width 0.03) (layer "F.Cu") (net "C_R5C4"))
 (segment (start 88.403449 93.918882) (end 89.110556 94.625988) (width 0.03) (layer "F.Cu") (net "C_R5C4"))
 (segment (start 100.707107 100.424264) (end 100.848528 100.565685) (width 0.03) (layer "F.Cu") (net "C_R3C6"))
 (segment (start 100.282843 100.848528) (end 100.707107 100.424264) (width 0.03) (layer "F.Cu") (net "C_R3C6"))
 (segment (start 89.676241 94.060303) (end 95.050253 95.615938) (width 0.03) (layer "F.Cu") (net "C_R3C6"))
 (segment (start 95.050253 95.615938) (end 100.282843 100.848528) (width 0.03) (layer "F.Cu") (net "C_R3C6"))
 (segment (start 88.969134 93.353196) (end 89.676241 94.060303) (width 0.03) (layer "F.Cu") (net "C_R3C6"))
 (segment (start 102.545584 97.737258) (end 102.828427 98.020101) (width 0.03) (layer "F.Cu") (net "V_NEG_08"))
 (segment (start 102.262742 97.454416) (end 102.545584 97.737258) (width 0.03) (layer "F.Cu") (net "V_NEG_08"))
 (segment (start 97.737258 92.928932) (end 101.697056 96.88873) (width 0.03) (layer "F.Cu") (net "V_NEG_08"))
 (segment (start 101.697056 96.88873) (end 101.979899 97.171573) (width 0.03) (layer "F.Cu") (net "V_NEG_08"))
 (segment (start 92.080404 90.241926) (end 92.787511 90.949033) (width 0.03) (layer "F.Cu") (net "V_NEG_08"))
 (segment (start 102.828427 98.020101) (end 103.11127 98.302944) (width 0.03) (layer "F.Cu") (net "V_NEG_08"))
 (segment (start 101.979899 97.171573) (end 102.262742 97.454416) (width 0.03) (layer "F.Cu") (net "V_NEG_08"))
 (segment (start 92.787511 90.949033) (end 97.737258 92.928932) (width 0.03) (layer "F.Cu") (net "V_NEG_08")))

